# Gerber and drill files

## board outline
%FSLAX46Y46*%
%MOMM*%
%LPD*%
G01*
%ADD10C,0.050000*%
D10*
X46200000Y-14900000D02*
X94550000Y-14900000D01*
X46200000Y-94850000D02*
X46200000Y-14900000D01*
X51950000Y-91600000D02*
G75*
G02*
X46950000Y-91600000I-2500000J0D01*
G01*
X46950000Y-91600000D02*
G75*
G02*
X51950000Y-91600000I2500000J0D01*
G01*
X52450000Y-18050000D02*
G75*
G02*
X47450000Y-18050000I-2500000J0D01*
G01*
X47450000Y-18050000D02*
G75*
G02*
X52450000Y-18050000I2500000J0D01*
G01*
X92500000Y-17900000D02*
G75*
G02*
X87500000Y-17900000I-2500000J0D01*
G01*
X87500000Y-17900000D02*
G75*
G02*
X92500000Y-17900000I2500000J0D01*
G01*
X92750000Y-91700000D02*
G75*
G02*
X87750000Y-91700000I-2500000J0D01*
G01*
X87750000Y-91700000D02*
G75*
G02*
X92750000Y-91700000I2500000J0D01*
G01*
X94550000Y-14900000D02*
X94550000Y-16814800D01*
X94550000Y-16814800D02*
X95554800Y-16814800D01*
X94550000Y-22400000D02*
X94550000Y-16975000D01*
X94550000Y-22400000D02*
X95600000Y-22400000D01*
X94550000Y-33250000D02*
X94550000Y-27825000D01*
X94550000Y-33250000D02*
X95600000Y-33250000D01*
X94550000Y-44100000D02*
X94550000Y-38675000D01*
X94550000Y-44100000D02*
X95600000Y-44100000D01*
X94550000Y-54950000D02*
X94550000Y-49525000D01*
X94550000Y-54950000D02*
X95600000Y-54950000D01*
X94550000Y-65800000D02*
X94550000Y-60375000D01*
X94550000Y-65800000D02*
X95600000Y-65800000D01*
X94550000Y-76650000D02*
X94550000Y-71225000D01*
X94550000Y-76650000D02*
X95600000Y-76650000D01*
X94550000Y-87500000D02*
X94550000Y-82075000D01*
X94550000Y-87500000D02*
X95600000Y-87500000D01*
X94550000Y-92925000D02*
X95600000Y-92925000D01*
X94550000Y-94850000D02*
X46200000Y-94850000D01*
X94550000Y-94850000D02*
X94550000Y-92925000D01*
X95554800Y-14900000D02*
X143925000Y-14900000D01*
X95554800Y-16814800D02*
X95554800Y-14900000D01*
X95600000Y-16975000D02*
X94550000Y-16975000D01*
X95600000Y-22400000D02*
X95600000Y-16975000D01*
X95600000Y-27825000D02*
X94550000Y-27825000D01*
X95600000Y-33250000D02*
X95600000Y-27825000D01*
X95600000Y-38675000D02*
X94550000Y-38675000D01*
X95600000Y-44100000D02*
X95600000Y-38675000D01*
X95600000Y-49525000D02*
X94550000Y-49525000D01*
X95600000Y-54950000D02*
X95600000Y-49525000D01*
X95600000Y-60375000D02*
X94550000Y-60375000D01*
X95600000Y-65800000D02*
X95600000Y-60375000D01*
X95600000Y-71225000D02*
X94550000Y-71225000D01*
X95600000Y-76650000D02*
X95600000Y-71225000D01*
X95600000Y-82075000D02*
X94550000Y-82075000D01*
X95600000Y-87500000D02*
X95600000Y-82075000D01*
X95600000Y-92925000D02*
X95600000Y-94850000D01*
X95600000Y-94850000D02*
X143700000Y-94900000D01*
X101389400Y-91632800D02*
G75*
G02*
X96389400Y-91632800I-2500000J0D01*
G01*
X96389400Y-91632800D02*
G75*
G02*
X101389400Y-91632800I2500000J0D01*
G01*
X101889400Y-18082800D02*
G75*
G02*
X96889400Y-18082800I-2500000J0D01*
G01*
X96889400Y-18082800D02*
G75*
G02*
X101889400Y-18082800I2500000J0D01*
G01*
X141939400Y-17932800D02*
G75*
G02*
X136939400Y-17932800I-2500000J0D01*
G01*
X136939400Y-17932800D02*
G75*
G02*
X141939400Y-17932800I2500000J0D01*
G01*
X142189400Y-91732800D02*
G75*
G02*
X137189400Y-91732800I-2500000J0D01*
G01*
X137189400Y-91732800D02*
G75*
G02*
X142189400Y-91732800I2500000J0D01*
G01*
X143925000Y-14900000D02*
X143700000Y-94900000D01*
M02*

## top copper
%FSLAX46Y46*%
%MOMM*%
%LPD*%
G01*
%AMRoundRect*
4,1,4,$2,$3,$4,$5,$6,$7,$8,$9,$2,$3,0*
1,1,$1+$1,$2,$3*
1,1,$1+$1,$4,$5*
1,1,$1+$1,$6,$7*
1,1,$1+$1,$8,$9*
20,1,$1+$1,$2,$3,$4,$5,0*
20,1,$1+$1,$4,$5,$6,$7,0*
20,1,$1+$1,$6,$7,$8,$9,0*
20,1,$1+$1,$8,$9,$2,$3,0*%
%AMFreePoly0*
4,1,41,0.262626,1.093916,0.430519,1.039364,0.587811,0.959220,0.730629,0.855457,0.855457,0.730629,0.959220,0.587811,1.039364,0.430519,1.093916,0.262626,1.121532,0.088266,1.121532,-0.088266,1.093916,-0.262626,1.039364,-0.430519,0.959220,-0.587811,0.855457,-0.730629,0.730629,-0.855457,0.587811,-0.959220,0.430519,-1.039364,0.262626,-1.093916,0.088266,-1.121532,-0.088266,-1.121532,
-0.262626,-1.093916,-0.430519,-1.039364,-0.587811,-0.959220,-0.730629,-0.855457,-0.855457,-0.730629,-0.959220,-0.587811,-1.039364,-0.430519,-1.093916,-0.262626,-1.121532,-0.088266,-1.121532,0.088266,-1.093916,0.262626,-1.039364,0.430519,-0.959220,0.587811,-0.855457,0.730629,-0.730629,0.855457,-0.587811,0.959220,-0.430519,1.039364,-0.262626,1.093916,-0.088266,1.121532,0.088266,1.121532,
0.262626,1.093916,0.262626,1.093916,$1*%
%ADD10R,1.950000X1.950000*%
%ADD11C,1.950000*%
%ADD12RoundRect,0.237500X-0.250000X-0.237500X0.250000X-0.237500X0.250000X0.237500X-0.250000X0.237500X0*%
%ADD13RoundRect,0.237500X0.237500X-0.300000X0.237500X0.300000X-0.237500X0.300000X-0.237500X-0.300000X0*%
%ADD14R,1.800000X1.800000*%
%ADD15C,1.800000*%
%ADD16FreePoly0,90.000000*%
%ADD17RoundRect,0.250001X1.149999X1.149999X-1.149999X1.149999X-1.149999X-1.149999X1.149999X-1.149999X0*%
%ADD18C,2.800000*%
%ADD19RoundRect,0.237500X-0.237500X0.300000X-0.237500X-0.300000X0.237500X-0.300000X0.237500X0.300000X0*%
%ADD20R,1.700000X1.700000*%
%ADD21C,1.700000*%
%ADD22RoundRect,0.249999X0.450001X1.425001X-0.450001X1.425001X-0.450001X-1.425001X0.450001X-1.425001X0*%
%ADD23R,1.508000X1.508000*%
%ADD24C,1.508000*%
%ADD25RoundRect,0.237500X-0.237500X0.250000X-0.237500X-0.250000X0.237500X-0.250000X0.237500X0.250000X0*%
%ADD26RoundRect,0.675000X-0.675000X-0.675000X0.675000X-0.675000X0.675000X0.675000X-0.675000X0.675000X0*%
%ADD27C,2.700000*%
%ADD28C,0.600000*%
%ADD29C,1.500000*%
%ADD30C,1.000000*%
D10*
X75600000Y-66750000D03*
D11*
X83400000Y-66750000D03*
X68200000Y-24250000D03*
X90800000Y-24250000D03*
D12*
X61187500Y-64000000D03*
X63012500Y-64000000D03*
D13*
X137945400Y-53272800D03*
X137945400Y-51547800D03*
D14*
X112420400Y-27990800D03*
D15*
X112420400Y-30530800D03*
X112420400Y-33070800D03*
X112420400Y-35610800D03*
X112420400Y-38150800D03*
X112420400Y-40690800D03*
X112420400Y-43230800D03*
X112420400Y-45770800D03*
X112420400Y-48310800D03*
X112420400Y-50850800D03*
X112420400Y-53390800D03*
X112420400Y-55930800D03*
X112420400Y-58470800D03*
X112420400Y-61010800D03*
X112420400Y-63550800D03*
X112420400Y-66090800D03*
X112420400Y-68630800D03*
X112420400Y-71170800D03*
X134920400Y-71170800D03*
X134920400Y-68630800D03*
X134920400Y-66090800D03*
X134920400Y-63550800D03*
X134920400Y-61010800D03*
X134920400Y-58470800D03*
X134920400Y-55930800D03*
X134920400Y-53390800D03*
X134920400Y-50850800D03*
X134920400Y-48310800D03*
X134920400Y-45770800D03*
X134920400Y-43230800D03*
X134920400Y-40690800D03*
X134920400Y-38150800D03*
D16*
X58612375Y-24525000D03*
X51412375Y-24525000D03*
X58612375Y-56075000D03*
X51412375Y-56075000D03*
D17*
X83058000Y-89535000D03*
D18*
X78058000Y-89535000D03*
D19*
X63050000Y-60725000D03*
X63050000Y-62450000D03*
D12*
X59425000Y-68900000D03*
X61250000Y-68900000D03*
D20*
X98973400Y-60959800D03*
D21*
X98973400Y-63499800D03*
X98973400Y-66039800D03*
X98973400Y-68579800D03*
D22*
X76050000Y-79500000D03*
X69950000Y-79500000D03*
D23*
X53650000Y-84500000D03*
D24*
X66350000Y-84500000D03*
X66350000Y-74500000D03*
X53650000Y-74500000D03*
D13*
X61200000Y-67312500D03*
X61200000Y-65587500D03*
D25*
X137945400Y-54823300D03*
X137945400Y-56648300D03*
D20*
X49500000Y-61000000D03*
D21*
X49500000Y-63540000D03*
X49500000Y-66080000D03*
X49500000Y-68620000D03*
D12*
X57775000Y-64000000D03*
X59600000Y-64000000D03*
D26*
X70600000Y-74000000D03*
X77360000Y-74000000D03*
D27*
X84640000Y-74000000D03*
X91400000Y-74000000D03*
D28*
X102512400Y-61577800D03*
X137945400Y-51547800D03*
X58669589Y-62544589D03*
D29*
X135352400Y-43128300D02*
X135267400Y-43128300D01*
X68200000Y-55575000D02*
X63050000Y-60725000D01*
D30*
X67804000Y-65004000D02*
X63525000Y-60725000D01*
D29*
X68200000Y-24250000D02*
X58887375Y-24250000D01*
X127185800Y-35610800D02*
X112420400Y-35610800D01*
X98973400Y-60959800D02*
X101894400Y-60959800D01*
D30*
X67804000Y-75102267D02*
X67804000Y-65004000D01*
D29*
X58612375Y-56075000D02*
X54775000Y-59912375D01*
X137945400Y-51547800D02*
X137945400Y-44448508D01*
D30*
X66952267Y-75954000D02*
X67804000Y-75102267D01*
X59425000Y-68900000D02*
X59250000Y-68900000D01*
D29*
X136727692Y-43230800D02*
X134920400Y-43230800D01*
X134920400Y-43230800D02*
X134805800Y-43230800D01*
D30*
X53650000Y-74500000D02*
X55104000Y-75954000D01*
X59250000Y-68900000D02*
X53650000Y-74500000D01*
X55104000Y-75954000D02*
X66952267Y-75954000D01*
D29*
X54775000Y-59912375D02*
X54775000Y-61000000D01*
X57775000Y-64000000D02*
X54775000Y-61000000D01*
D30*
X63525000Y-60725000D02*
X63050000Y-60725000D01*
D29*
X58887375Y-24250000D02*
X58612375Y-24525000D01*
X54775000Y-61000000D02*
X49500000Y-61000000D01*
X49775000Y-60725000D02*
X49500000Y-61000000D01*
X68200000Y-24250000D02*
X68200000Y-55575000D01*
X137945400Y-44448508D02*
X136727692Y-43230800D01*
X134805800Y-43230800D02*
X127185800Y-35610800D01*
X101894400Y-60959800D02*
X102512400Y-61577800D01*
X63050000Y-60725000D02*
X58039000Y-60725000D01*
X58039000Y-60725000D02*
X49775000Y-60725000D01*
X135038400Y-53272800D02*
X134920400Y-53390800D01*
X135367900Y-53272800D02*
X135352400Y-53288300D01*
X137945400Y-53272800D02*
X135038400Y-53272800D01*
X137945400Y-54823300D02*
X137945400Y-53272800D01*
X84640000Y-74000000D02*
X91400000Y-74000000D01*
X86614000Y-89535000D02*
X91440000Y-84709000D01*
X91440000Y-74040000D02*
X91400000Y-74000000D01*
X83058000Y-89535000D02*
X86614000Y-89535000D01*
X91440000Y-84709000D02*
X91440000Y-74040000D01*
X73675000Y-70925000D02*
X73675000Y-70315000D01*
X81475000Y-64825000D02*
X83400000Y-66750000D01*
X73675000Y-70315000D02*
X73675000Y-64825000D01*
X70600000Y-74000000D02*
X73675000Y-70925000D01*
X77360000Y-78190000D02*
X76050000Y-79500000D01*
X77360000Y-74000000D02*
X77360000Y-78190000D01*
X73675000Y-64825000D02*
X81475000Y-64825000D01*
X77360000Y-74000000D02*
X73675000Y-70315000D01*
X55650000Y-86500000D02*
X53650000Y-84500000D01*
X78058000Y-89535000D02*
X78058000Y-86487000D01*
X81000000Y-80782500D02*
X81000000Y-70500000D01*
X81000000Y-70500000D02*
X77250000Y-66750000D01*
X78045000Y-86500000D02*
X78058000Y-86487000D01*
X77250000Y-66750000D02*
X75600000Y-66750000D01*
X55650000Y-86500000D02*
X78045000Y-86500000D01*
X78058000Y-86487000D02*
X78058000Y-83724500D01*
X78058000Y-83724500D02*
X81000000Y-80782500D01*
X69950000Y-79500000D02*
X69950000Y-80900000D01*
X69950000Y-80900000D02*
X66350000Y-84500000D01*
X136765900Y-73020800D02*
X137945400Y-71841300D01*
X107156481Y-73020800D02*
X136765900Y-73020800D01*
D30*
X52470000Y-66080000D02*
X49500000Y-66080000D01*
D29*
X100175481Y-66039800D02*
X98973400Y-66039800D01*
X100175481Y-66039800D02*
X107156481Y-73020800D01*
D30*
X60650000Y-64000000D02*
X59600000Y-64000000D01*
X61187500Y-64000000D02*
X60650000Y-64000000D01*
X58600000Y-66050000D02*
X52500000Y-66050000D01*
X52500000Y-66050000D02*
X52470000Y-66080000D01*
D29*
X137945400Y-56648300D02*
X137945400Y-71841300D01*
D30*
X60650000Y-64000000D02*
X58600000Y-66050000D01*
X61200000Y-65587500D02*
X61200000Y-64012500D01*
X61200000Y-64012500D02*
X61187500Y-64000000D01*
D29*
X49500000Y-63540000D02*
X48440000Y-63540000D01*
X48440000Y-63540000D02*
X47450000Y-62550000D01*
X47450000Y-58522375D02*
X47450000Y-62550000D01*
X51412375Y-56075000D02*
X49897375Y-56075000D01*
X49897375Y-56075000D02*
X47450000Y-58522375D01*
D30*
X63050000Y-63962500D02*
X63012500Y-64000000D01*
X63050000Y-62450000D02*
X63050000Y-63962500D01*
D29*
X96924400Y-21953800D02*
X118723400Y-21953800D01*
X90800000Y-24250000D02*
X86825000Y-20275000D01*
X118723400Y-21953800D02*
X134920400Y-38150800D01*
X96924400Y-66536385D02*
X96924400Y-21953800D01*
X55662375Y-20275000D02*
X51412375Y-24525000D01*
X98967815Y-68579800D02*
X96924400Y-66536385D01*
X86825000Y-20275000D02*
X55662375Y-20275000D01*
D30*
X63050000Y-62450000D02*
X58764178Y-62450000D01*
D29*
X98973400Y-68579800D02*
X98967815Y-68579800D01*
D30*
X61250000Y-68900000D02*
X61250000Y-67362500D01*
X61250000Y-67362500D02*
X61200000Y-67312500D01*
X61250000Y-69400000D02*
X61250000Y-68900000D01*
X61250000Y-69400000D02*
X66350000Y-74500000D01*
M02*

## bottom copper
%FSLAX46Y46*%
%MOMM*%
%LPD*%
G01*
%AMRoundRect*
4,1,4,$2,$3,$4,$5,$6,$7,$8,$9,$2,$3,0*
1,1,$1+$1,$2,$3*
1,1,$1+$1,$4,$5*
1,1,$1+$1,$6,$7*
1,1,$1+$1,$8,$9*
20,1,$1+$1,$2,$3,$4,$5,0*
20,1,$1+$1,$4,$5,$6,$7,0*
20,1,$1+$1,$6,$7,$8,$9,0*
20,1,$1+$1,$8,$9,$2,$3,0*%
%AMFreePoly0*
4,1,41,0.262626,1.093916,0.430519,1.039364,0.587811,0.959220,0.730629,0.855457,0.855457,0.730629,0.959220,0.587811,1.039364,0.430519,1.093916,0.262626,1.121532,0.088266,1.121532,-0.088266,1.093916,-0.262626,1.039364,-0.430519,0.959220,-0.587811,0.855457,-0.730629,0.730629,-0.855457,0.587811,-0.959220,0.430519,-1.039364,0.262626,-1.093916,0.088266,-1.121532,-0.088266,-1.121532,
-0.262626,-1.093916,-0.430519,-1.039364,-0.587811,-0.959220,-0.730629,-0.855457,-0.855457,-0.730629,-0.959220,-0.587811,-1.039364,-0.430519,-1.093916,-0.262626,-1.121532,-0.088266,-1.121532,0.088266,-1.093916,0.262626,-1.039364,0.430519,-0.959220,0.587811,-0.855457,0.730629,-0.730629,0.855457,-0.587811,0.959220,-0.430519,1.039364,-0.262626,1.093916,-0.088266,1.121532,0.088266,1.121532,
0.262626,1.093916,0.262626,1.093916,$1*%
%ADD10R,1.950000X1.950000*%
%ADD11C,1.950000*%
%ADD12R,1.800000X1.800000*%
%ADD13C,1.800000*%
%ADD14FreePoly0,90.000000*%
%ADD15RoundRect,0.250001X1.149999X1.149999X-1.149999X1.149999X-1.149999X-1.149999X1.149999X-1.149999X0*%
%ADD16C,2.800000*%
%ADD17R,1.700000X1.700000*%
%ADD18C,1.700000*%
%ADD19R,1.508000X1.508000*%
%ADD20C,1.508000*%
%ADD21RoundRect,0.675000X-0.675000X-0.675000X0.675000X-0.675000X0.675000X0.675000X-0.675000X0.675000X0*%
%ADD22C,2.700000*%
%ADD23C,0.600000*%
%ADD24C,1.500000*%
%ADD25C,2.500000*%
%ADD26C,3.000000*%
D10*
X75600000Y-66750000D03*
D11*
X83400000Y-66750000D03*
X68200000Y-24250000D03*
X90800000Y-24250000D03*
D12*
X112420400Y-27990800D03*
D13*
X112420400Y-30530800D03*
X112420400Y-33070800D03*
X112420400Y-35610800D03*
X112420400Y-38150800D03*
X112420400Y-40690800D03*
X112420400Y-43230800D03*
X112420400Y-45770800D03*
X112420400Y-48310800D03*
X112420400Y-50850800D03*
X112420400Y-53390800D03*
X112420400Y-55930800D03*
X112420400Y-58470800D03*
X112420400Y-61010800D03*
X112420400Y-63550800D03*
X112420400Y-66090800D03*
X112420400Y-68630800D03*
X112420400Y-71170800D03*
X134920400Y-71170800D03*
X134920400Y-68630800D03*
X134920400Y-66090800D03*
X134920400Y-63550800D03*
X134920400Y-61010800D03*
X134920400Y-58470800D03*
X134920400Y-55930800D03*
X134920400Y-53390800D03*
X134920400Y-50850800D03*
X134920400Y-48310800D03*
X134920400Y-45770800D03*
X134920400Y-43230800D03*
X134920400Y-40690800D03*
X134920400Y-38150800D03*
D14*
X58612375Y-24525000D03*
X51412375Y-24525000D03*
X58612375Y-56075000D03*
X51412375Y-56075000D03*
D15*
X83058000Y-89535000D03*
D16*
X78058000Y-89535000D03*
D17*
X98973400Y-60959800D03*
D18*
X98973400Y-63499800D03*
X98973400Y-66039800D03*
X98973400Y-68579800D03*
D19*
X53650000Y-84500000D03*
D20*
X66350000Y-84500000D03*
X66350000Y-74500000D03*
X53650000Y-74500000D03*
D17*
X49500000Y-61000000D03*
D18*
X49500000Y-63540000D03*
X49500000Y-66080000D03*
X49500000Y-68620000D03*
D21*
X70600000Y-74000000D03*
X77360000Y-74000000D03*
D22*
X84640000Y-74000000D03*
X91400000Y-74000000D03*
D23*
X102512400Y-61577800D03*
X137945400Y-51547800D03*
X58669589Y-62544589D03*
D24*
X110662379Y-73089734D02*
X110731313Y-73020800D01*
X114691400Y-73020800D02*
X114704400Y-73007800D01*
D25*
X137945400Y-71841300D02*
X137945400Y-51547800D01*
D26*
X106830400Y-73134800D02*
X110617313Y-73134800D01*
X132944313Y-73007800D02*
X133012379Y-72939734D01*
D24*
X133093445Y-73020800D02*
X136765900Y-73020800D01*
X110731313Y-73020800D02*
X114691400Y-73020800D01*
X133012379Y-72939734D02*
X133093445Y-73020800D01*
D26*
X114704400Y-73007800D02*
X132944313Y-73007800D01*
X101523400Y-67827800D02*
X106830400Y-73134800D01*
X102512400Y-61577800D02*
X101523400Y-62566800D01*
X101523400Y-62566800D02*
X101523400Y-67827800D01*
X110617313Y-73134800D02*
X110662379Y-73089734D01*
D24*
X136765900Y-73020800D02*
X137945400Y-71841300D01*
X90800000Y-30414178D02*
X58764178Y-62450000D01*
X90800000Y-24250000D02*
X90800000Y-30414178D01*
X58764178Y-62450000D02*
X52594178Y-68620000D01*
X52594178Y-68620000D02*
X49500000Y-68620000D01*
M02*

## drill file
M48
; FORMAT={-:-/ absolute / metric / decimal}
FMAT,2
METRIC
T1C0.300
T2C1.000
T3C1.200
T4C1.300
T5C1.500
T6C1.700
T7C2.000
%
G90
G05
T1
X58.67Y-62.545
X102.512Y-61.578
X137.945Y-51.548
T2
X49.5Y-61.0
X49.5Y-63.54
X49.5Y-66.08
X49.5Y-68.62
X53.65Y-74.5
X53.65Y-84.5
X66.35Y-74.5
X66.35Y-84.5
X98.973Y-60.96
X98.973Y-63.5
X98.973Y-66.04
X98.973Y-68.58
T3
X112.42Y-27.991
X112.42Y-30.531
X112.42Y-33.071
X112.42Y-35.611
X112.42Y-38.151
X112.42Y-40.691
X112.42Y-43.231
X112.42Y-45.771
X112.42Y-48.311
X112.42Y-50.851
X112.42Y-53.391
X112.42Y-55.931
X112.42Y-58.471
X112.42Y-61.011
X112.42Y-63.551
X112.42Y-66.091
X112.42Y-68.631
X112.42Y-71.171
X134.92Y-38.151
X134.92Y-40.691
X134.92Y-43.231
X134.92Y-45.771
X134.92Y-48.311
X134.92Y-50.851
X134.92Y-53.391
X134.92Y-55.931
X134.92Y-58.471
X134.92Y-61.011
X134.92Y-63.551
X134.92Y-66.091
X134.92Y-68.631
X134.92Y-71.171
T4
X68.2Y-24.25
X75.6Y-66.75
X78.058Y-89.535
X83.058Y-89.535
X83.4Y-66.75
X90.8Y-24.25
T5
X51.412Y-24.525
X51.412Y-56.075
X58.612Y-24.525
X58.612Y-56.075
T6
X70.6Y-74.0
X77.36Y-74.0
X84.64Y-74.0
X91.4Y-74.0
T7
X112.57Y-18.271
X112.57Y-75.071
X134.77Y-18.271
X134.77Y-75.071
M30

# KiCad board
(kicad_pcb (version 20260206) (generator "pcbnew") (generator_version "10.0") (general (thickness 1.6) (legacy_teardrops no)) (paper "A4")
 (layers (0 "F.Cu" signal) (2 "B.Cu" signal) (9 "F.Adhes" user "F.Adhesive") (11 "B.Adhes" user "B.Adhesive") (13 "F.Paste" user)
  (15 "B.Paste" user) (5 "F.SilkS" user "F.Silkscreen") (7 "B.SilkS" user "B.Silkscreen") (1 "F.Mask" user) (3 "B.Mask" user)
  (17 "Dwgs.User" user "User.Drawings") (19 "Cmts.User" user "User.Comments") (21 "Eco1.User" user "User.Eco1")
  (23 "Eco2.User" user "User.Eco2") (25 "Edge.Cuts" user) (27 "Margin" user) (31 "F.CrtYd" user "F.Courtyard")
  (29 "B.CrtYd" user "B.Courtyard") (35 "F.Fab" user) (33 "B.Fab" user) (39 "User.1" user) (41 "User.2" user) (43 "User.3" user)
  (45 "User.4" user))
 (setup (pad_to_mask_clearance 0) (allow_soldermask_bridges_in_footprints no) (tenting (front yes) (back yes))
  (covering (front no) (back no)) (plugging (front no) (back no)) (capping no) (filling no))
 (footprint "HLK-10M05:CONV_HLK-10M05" (layer "F.Cu") (at 79.5 45.5 90)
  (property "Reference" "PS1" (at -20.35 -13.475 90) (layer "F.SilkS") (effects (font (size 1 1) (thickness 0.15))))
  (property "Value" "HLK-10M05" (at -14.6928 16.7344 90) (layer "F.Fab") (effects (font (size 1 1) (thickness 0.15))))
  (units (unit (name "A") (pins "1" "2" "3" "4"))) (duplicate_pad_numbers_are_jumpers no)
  (pad "1" thru_hole rect (at -21.25 -3.9 90) (size 1.95 1.95) (drill 1.3) (layers "*.Cu" "*.Mask") (remove_unused_layers no) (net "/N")
   (solder_mask_margin 0.102))
  (pad "2" thru_hole circle (at -21.25 3.9 90) (size 1.95 1.95) (drill 1.3) (layers "*.Cu" "*.Mask") (remove_unused_layers no)
   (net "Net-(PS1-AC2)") (solder_mask_margin 0.102))
  (pad "3" thru_hole circle (at 21.25 -11.3 90) (size 1.95 1.95) (drill 1.3) (layers "*.Cu" "*.Mask") (remove_unused_layers no) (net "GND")
   (solder_mask_margin 0.102))
  (pad "4" thru_hole circle (at 21.25 11.3 90) (size 1.95 1.95) (drill 1.3) (layers "*.Cu" "*.Mask") (remove_unused_layers no) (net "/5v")
   (solder_mask_margin 0.102)))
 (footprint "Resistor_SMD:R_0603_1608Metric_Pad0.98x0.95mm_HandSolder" (layer "F.Cu") (at 62.1 64)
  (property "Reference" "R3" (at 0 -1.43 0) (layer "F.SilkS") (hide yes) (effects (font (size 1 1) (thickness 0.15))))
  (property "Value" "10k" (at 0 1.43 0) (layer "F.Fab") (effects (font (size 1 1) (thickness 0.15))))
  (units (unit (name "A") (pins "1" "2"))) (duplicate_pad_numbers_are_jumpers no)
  (pad "1" smd roundrect (at -0.9125 0) (size 0.975 0.95) (layers "F.Cu" "F.Mask" "F.Paste") (roundrect_rratio 0.25) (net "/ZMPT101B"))
  (pad "2" smd roundrect (at 0.9125 0) (size 0.975 0.95) (layers "F.Cu" "F.Mask" "F.Paste") (roundrect_rratio 0.25) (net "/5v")))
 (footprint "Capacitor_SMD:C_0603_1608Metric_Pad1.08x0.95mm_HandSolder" (layer "F.Cu") (at 137.9454 52.4103 90)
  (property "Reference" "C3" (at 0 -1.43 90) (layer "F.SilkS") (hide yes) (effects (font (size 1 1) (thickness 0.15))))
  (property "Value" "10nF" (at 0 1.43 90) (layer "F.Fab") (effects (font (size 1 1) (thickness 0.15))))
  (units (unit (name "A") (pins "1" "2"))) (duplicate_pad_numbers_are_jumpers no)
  (pad "1" smd roundrect (at -0.8625 0 90) (size 1.075 0.95) (layers "F.Cu" "F.Mask" "F.Paste") (roundrect_rratio 0.25) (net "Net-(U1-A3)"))
  (pad "2" smd roundrect (at 0.8625 0 90) (size 1.075 0.95) (layers "F.Cu" "F.Mask" "F.Paste") (roundrect_rratio 0.25) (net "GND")))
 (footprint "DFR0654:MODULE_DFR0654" (layer "F.Cu") (at 123.6704 46.6708)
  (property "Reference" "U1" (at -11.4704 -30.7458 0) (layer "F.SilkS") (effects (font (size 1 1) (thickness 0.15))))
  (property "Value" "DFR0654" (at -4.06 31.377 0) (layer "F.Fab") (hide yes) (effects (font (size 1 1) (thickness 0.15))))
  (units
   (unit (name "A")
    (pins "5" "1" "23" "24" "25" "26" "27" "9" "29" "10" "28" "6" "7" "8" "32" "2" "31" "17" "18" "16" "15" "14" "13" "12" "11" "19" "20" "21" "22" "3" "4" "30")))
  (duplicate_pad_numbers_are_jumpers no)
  (pad "" np_thru_hole circle (at -11.1 -28.4) (size 2 2) (drill 2) (layers "*.Cu" "*.Mask"))
  (pad "" np_thru_hole circle (at -11.1 28.4) (size 2 2) (drill 2) (layers "*.Cu" "*.Mask"))
  (pad "" np_thru_hole circle (at 11.1 -28.4) (size 2 2) (drill 2) (layers "*.Cu" "*.Mask"))
  (pad "" np_thru_hole circle (at 11.1 28.4) (size 2 2) (drill 2) (layers "*.Cu" "*.Mask"))
  (pad "1" thru_hole rect (at -11.25 -18.68) (size 1.8 1.8) (drill 1.2) (layers "*.Cu" "*.Mask") (remove_unused_layers no)
   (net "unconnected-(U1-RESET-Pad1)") (solder_mask_margin 0.102))
  (pad "2" thru_hole circle (at -11.25 -16.14) (size 1.8 1.8) (drill 1.2) (layers "*.Cu" "*.Mask") (remove_unused_layers no) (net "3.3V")
   (solder_mask_margin 0.102))
  (pad "3" thru_hole circle (at -11.25 -13.6) (size 1.8 1.8) (drill 1.2) (layers "*.Cu" "*.Mask") (remove_unused_layers no)
   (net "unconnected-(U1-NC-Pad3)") (solder_mask_margin 0.102))
  (pad "4" thru_hole circle (at -11.25 -11.06) (size 1.8 1.8) (drill 1.2) (layers "*.Cu" "*.Mask") (remove_unused_layers no) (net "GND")
   (solder_mask_margin 0.102))
  (pad "5" thru_hole circle (at -11.25 -8.52) (size 1.8 1.8) (drill 1.2) (layers "*.Cu" "*.Mask") (remove_unused_layers no)
   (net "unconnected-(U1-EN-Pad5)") (solder_mask_margin 0.102))
  (pad "6" thru_hole circle (at -11.25 -5.98) (size 1.8 1.8) (drill 1.2) (layers "*.Cu" "*.Mask") (remove_unused_layers no)
   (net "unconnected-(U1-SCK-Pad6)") (solder_mask_margin 0.102))
  (pad "7" thru_hole circle (at -11.25 -3.44) (size 1.8 1.8) (drill 1.2) (layers "*.Cu" "*.Mask") (remove_unused_layers no)
   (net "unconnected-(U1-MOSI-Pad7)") (solder_mask_margin 0.102))
  (pad "8" thru_hole circle (at -11.25 -0.9) (size 1.8 1.8) (drill 1.2) (layers "*.Cu" "*.Mask") (remove_unused_layers no)
   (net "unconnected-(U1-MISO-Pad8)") (solder_mask_margin 0.102))
  (pad "9" thru_hole circle (at -11.25 1.64) (size 1.8 1.8) (drill 1.2) (layers "*.Cu" "*.Mask") (remove_unused_layers no)
   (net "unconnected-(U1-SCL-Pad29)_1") (solder_mask_margin 0.102))
  (pad "10" thru_hole circle (at -11.25 4.18) (size 1.8 1.8) (drill 1.2) (layers "*.Cu" "*.Mask") (remove_unused_layers no)
   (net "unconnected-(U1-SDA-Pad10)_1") (solder_mask_margin 0.102))
  (pad "11" thru_hole circle (at -11.25 6.72) (size 1.8 1.8) (drill 1.2) (layers "*.Cu" "*.Mask") (remove_unused_layers no)
   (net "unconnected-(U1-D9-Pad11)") (solder_mask_margin 0.102))
  (pad "12" thru_hole circle (at -11.25 9.26) (size 1.8 1.8) (drill 1.2) (layers "*.Cu" "*.Mask") (remove_unused_layers no)
   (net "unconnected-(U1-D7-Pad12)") (solder_mask_margin 0.102))
  (pad "13" thru_hole circle (at -11.25 11.8) (size 1.8 1.8) (drill 1.2) (layers "*.Cu" "*.Mask") (remove_unused_layers no)
   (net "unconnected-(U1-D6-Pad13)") (solder_mask_margin 0.102))
  (pad "14" thru_hole circle (at -11.25 14.34) (size 1.8 1.8) (drill 1.2) (layers "*.Cu" "*.Mask") (remove_unused_layers no)
   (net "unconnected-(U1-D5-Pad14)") (solder_mask_margin 0.102))
  (pad "15" thru_hole circle (at -11.25 16.88) (size 1.8 1.8) (drill 1.2) (layers "*.Cu" "*.Mask") (remove_unused_layers no)
   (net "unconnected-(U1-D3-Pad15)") (solder_mask_margin 0.102))
  (pad "16" thru_hole circle (at -11.25 19.42) (size 1.8 1.8) (drill 1.2) (layers "*.Cu" "*.Mask") (remove_unused_layers no)
   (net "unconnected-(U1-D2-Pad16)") (solder_mask_margin 0.102))
  (pad "17" thru_hole circle (at -11.25 21.96) (size 1.8 1.8) (drill 1.2) (layers "*.Cu" "*.Mask") (remove_unused_layers no)
   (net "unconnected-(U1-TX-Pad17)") (solder_mask_margin 0.102))
  (pad "18" thru_hole circle (at -11.25 24.5) (size 1.8 1.8) (drill 1.2) (layers "*.Cu" "*.Mask") (remove_unused_layers no)
   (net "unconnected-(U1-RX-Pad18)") (solder_mask_margin 0.102))
  (pad "19" thru_hole circle (at 11.25 24.5) (size 1.8 1.8) (drill 1.2) (layers "*.Cu" "*.Mask") (remove_unused_layers no)
   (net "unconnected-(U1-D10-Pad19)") (solder_mask_margin 0.102))
  (pad "20" thru_hole circle (at 11.25 21.96) (size 1.8 1.8) (drill 1.2) (layers "*.Cu" "*.Mask") (remove_unused_layers no)
   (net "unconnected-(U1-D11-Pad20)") (solder_mask_margin 0.102))
  (pad "21" thru_hole circle (at 11.25 19.42) (size 1.8 1.8) (drill 1.2) (layers "*.Cu" "*.Mask") (remove_unused_layers no)
   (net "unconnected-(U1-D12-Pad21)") (solder_mask_margin 0.102))
  (pad "22" thru_hole circle (at 11.25 16.88) (size 1.8 1.8) (drill 1.2) (layers "*.Cu" "*.Mask") (remove_unused_layers no)
   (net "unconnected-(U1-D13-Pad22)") (solder_mask_margin 0.102))
  (pad "23" thru_hole circle (at 11.25 14.34) (size 1.8 1.8) (drill 1.2) (layers "*.Cu" "*.Mask") (remove_unused_layers no)
   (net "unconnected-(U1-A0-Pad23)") (solder_mask_margin 0.102))
  (pad "24" thru_hole circle (at 11.25 11.8) (size 1.8 1.8) (drill 1.2) (layers "*.Cu" "*.Mask") (remove_unused_layers no)
   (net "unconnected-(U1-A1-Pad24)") (solder_mask_margin 0.102))
  (pad "25" thru_hole circle (at 11.25 9.26) (size 1.8 1.8) (drill 1.2) (layers "*.Cu" "*.Mask") (remove_unused_layers no)
   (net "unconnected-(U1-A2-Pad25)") (solder_mask_margin 0.102))
  (pad "26" thru_hole circle (at 11.25 6.72) (size 1.8 1.8) (drill 1.2) (layers "*.Cu" "*.Mask") (remove_unused_layers no)
   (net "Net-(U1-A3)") (solder_mask_margin 0.102))
  (pad "27" thru_hole circle (at 11.25 4.18) (size 1.8 1.8) (drill 1.2) (layers "*.Cu" "*.Mask") (remove_unused_layers no)
   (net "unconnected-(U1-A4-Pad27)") (solder_mask_margin 0.102))
  (pad "28" thru_hole circle (at 11.25 1.64) (size 1.8 1.8) (drill 1.2) (layers "*.Cu" "*.Mask") (remove_unused_layers no)
   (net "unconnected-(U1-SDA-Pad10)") (solder_mask_margin 0.102))
  (pad "29" thru_hole circle (at 11.25 -0.9) (size 1.8 1.8) (drill 1.2) (layers "*.Cu" "*.Mask") (remove_unused_layers no)
   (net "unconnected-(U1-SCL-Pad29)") (solder_mask_margin 0.102))
  (pad "30" thru_hole circle (at 11.25 -3.44) (size 1.8 1.8) (drill 1.2) (layers "*.Cu" "*.Mask") (remove_unused_layers no) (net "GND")
   (solder_mask_margin 0.102))
  (pad "31" thru_hole circle (at 11.25 -5.98) (size 1.8 1.8) (drill 1.2) (layers "*.Cu" "*.Mask") (remove_unused_layers no) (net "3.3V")
   (solder_mask_margin 0.102))
  (pad "32" thru_hole circle (at 11.25 -8.52) (size 1.8 1.8) (drill 1.2) (layers "*.Cu" "*.Mask") (remove_unused_layers no) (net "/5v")
   (solder_mask_margin 0.102)))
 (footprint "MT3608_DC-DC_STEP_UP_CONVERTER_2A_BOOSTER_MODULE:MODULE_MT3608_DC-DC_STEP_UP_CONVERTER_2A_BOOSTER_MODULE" (layer "F.Cu")
  (at 55.012375 40.3 90)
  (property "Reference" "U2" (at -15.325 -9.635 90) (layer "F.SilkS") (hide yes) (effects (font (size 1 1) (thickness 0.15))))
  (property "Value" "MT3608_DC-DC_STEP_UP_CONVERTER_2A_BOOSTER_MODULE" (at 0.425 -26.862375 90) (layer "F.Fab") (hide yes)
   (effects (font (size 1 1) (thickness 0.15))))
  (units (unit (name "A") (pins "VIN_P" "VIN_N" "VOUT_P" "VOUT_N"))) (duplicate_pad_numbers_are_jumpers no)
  (pad "VIN_N" thru_hole custom (at 15.775 3.6 90) (size 2.25 2.25) (drill 1.5) (layers "*.Cu") (remove_unused_layers no) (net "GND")
   (thermal_bridge_angle 90) (options (clearance outline) (anchor circle)) (primitives))
  (pad "VIN_P" thru_hole custom (at 15.775 -3.6 90) (size 2.25 2.25) (drill 1.5) (layers "*.Cu") (remove_unused_layers no) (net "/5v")
   (thermal_bridge_angle 90) (options (clearance outline) (anchor circle)) (primitives))
  (pad "VOUT_N" thru_hole custom (at -15.775 3.6 90) (size 2.25 2.25) (drill 1.5) (layers "*.Cu") (remove_unused_layers no) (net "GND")
   (thermal_bridge_angle 90) (options (clearance outline) (anchor circle)) (primitives))
  (pad "VOUT_P" thru_hole custom (at -15.775 -3.6 90) (size 2.25 2.25) (drill 1.5) (layers "*.Cu") (remove_unused_layers no) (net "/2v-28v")
   (thermal_bridge_angle 90) (options (clearance outline) (anchor circle)) (primitives)))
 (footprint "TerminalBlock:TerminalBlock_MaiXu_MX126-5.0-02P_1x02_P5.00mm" (layer "F.Cu") (at 83.058 89.535 180)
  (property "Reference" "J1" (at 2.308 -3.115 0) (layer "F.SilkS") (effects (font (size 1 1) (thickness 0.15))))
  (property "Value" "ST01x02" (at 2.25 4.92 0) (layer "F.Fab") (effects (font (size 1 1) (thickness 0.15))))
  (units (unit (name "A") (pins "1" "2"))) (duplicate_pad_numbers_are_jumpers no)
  (pad "1" thru_hole roundrect (at 0 0 180) (size 2.8 2.8) (drill 1.3) (layers "*.Cu" "*.Mask") (remove_unused_layers no)
   (roundrect_rratio 0.089286) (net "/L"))
  (pad "2" thru_hole circle (at 5 0 180) (size 2.8 2.8) (drill 1.3) (layers "*.Cu" "*.Mask") (remove_unused_layers no) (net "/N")))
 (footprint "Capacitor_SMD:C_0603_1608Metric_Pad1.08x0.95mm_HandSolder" (layer "F.Cu") (at 63.05 61.5875 -90)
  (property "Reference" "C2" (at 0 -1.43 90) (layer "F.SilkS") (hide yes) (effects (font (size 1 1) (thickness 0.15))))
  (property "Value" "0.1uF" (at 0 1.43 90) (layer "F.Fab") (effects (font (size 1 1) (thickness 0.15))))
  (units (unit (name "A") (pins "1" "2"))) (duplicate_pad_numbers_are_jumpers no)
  (pad "1" smd roundrect (at -0.8625 0 270) (size 1.075 0.95) (layers "F.Cu" "F.Mask" "F.Paste") (roundrect_rratio 0.25) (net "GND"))
  (pad "2" smd roundrect (at 0.8625 0 270) (size 1.075 0.95) (layers "F.Cu" "F.Mask" "F.Paste") (roundrect_rratio 0.25) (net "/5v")))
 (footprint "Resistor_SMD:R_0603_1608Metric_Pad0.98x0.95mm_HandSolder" (layer "F.Cu") (at 60.3375 68.9)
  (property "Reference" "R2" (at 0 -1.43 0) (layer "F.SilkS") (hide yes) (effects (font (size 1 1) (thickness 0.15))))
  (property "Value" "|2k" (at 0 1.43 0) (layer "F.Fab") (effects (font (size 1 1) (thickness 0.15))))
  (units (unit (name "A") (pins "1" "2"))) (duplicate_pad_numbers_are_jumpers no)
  (pad "1" smd roundrect (at -0.9125 0) (size 0.975 0.95) (layers "F.Cu" "F.Mask" "F.Paste") (roundrect_rratio 0.25) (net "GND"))
  (pad "2" smd roundrect (at 0.9125 0) (size 0.975 0.95) (layers "F.Cu" "F.Mask" "F.Paste") (roundrect_rratio 0.25) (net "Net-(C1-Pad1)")))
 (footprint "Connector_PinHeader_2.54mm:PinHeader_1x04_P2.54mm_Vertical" (layer "F.Cu") (at 98.9734 60.9598)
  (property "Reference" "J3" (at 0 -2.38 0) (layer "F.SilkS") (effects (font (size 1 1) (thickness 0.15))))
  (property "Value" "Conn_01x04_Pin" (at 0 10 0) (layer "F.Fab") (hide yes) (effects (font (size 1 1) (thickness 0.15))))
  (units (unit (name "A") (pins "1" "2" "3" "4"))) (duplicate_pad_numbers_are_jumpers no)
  (pad "1" thru_hole rect (at 0 0) (size 1.7 1.7) (drill 1) (layers "*.Cu" "*.Mask") (remove_unused_layers no) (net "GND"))
  (pad "2" thru_hole circle (at 0 2.54) (size 1.7 1.7) (drill 1) (layers "*.Cu" "*.Mask") (remove_unused_layers no)
   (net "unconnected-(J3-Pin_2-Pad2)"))
  (pad "3" thru_hole circle (at 0 5.08) (size 1.7 1.7) (drill 1) (layers "*.Cu" "*.Mask") (remove_unused_layers no) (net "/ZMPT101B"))
  (pad "4" thru_hole circle (at 0 7.62) (size 1.7 1.7) (drill 1) (layers "*.Cu" "*.Mask") (remove_unused_layers no) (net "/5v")))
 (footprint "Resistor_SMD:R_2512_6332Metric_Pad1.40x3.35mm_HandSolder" (layer "F.Cu") (at 73 79.5 180)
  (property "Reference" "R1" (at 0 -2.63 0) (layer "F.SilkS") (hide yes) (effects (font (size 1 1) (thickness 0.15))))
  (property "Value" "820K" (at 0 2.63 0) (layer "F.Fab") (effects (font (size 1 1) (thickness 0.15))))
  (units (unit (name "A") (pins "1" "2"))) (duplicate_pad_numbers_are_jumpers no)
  (pad "1" smd roundrect (at -3.05 0 180) (size 1.4 3.35) (layers "F.Cu" "F.Mask" "F.Paste") (roundrect_rratio 0.178571)
   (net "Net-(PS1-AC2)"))
  (pad "2" smd roundrect (at 3.05 0 180) (size 1.4 3.35) (layers "F.Cu" "F.Mask" "F.Paste") (roundrect_rratio 0.178571)
   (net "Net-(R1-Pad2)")))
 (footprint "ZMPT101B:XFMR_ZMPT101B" (layer "F.Cu") (at 60 79.5 90)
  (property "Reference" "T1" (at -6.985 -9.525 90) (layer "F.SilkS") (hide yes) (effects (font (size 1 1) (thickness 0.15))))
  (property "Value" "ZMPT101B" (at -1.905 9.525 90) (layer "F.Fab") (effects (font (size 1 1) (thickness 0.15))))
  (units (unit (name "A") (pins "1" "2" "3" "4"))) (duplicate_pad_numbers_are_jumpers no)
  (pad "1" thru_hole rect (at -5 -6.35 90) (size 1.508 1.508) (drill 1) (layers "*.Cu" "*.Mask") (remove_unused_layers no) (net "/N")
   (solder_mask_margin 0.102))
  (pad "2" thru_hole circle (at -5 6.35 90) (size 1.508 1.508) (drill 1) (layers "*.Cu" "*.Mask") (remove_unused_layers no)
   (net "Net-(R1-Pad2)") (solder_mask_margin 0.102))
  (pad "3" thru_hole circle (at 5 6.35 90) (size 1.508 1.508) (drill 1) (layers "*.Cu" "*.Mask") (remove_unused_layers no)
   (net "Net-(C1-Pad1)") (solder_mask_margin 0.102))
  (pad "4" thru_hole circle (at 5 -6.35 90) (size 1.508 1.508) (drill 1) (layers "*.Cu" "*.Mask") (remove_unused_layers no) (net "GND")
   (solder_mask_margin 0.102)))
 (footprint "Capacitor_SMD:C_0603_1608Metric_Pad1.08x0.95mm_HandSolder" (layer "F.Cu") (at 61.2 66.45 90)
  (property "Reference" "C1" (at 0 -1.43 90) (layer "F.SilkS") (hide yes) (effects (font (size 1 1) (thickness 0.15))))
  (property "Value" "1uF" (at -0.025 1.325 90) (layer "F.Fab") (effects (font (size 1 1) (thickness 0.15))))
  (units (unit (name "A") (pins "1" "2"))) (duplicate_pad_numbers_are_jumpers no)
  (pad "1" smd roundrect (at -0.8625 0 90) (size 1.075 0.95) (layers "F.Cu" "F.Mask" "F.Paste") (roundrect_rratio 0.25)
   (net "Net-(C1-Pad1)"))
  (pad "2" smd roundrect (at 0.8625 0 90) (size 1.075 0.95) (layers "F.Cu" "F.Mask" "F.Paste") (roundrect_rratio 0.25) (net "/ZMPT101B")))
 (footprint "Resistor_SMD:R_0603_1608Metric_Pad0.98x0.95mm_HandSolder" (layer "F.Cu") (at 137.9454 55.7358 -90)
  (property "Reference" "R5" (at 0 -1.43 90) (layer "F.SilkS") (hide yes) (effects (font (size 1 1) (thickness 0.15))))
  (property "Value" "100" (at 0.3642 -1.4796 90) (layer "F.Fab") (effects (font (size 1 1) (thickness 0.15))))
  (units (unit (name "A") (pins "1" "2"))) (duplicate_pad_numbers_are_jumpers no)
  (pad "1" smd roundrect (at -0.9125 0 270) (size 0.975 0.95) (layers "F.Cu" "F.Mask" "F.Paste") (roundrect_rratio 0.25) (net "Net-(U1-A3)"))
  (pad "2" smd roundrect (at 0.9125 0 270) (size 0.975 0.95) (layers "F.Cu" "F.Mask" "F.Paste") (roundrect_rratio 0.25) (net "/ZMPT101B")))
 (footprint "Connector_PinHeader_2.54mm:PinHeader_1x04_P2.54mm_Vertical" (layer "F.Cu") (at 49.5 61)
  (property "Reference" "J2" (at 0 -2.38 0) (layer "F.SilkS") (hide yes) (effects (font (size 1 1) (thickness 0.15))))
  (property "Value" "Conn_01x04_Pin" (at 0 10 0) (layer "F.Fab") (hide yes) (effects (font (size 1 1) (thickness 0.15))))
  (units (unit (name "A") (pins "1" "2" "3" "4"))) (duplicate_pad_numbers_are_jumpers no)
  (pad "1" thru_hole rect (at 0 0) (size 1.7 1.7) (drill 1) (layers "*.Cu" "*.Mask") (remove_unused_layers no) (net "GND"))
  (pad "2" thru_hole circle (at 0 2.54) (size 1.7 1.7) (drill 1) (layers "*.Cu" "*.Mask") (remove_unused_layers no) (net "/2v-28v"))
  (pad "3" thru_hole circle (at 0 5.08) (size 1.7 1.7) (drill 1) (layers "*.Cu" "*.Mask") (remove_unused_layers no) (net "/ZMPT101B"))
  (pad "4" thru_hole circle (at 0 7.62) (size 1.7 1.7) (drill 1) (layers "*.Cu" "*.Mask") (remove_unused_layers no) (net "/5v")))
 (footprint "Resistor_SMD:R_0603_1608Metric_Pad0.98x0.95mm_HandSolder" (layer "F.Cu") (at 58.6875 64)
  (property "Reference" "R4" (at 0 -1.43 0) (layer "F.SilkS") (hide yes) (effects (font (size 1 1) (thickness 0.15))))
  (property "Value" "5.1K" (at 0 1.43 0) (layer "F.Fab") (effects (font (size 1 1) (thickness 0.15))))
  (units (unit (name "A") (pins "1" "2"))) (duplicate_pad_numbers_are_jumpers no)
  (pad "1" smd roundrect (at -0.9125 0) (size 0.975 0.95) (layers "F.Cu" "F.Mask" "F.Paste") (roundrect_rratio 0.25) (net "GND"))
  (pad "2" smd roundrect (at 0.9125 0) (size 0.975 0.95) (layers "F.Cu" "F.Mask" "F.Paste") (roundrect_rratio 0.25) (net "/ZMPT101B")))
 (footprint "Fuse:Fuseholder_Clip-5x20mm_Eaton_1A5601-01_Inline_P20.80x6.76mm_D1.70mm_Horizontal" (layer "F.Cu") (at 70.6 74)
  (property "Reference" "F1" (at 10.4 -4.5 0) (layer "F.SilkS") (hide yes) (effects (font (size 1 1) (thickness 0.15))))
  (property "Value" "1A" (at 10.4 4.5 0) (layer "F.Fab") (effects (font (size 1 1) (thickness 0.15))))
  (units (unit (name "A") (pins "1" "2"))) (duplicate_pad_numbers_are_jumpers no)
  (pad "1" thru_hole roundrect (at 0 0) (size 2.7 2.7) (drill 1.7) (layers "*.Cu" "*.Mask") (remove_unused_layers no)
   (roundrect_rratio 0.25) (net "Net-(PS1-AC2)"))
  (pad "1" thru_hole roundrect (at 6.76 0) (size 2.7 2.7) (drill 1.7) (layers "*.Cu" "*.Mask") (remove_unused_layers no)
   (roundrect_rratio 0.25) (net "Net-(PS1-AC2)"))
  (pad "2" thru_hole circle (at 14.04 0) (size 2.7 2.7) (drill 1.7) (layers "*.Cu" "*.Mask") (remove_unused_layers no) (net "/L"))
  (pad "2" thru_hole circle (at 20.8 0) (size 2.7 2.7) (drill 1.7) (layers "*.Cu" "*.Mask") (remove_unused_layers no) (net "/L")))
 (gr_line (start 46.2 14.9) (end 94.55 14.9) (stroke (width 0.05) (type default)) (layer "Edge.Cuts"))
 (gr_line (start 46.2 94.85) (end 46.2 14.9) (stroke (width 0.05) (type default)) (layer "Edge.Cuts"))
 (gr_circle (center 49.45 91.6) (end 51.95 91.6) (stroke (width 0.05) (type default)) (fill no) (layer "Edge.Cuts"))
 (gr_circle (center 49.95 18.05) (end 52.45 18.05) (stroke (width 0.05) (type default)) (fill no) (layer "Edge.Cuts"))
 (gr_circle (center 90 17.9) (end 92.5 17.9) (stroke (width 0.05) (type default)) (fill no) (layer "Edge.Cuts"))
 (gr_circle (center 90.25 91.7) (end 92.75 91.7) (stroke (width 0.05) (type default)) (fill no) (layer "Edge.Cuts"))
 (gr_line (start 94.55 14.9) (end 94.55 16.8148) (stroke (width 0.05) (type default)) (layer "Edge.Cuts"))
 (gr_line (start 94.55 16.8148) (end 95.5548 16.8148) (stroke (width 0.05) (type default)) (layer "Edge.Cuts"))
 (gr_line (start 94.55 22.4) (end 94.55 16.975) (stroke (width 0.05) (type default)) (layer "Edge.Cuts"))
 (gr_line (start 94.55 22.4) (end 95.6 22.4) (stroke (width 0.05) (type default)) (layer "Edge.Cuts"))
 (gr_line (start 94.55 33.25) (end 94.55 27.825) (stroke (width 0.05) (type default)) (layer "Edge.Cuts"))
 (gr_line (start 94.55 33.25) (end 95.6 33.25) (stroke (width 0.05) (type default)) (layer "Edge.Cuts"))
 (gr_line (start 94.55 44.1) (end 94.55 38.675) (stroke (width 0.05) (type default)) (layer "Edge.Cuts"))
 (gr_line (start 94.55 44.1) (end 95.6 44.1) (stroke (width 0.05) (type default)) (layer "Edge.Cuts"))
 (gr_line (start 94.55 54.95) (end 94.55 49.525) (stroke (width 0.05) (type default)) (layer "Edge.Cuts"))
 (gr_line (start 94.55 54.95) (end 95.6 54.95) (stroke (width 0.05) (type default)) (layer "Edge.Cuts"))
 (gr_line (start 94.55 65.8) (end 94.55 60.375) (stroke (width 0.05) (type default)) (layer "Edge.Cuts"))
 (gr_line (start 94.55 65.8) (end 95.6 65.8) (stroke (width 0.05) (type default)) (layer "Edge.Cuts"))
 (gr_line (start 94.55 76.65) (end 94.55 71.225) (stroke (width 0.05) (type default)) (layer "Edge.Cuts"))
 (gr_line (start 94.55 76.65) (end 95.6 76.65) (stroke (width 0.05) (type default)) (layer "Edge.Cuts"))
 (gr_line (start 94.55 87.5) (end 94.55 82.075) (stroke (width 0.05) (type default)) (layer "Edge.Cuts"))
 (gr_line (start 94.55 87.5) (end 95.6 87.5) (stroke (width 0.05) (type default)) (layer "Edge.Cuts"))
 (gr_line (start 94.55 92.925) (end 95.6 92.925) (stroke (width 0.05) (type default)) (layer "Edge.Cuts"))
 (gr_line (start 94.55 94.85) (end 46.2 94.85) (stroke (width 0.05) (type default)) (layer "Edge.Cuts"))
 (gr_line (start 94.55 94.85) (end 94.55 92.925) (stroke (width 0.05) (type default)) (layer "Edge.Cuts"))
 (gr_line (start 95.5548 14.9) (end 143.925 14.9) (stroke (width 0.05) (type default)) (layer "Edge.Cuts"))
 (gr_line (start 95.5548 16.8148) (end 95.5548 14.9) (stroke (width 0.05) (type default)) (layer "Edge.Cuts"))
 (gr_line (start 95.6 16.975) (end 94.55 16.975) (stroke (width 0.05) (type default)) (layer "Edge.Cuts"))
 (gr_line (start 95.6 22.4) (end 95.6 16.975) (stroke (width 0.05) (type default)) (layer "Edge.Cuts"))
 (gr_line (start 95.6 27.825) (end 94.55 27.825) (stroke (width 0.05) (type default)) (layer "Edge.Cuts"))
 (gr_line (start 95.6 33.25) (end 95.6 27.825) (stroke (width 0.05) (type default)) (layer "Edge.Cuts"))
 (gr_line (start 95.6 38.675) (end 94.55 38.675) (stroke (width 0.05) (type default)) (layer "Edge.Cuts"))
 (gr_line (start 95.6 44.1) (end 95.6 38.675) (stroke (width 0.05) (type default)) (layer "Edge.Cuts"))
 (gr_line (start 95.6 49.525) (end 94.55 49.525) (stroke (width 0.05) (type default)) (layer "Edge.Cuts"))
 (gr_line (start 95.6 54.95) (end 95.6 49.525) (stroke (width 0.05) (type default)) (layer "Edge.Cuts"))
 (gr_line (start 95.6 60.375) (end 94.55 60.375) (stroke (width 0.05) (type default)) (layer "Edge.Cuts"))
 (gr_line (start 95.6 65.8) (end 95.6 60.375) (stroke (width 0.05) (type default)) (layer "Edge.Cuts"))
 (gr_line (start 95.6 71.225) (end 94.55 71.225) (stroke (width 0.05) (type default)) (layer "Edge.Cuts"))
 (gr_line (start 95.6 76.65) (end 95.6 71.225) (stroke (width 0.05) (type default)) (layer "Edge.Cuts"))
 (gr_line (start 95.6 82.075) (end 94.55 82.075) (stroke (width 0.05) (type default)) (layer "Edge.Cuts"))
 (gr_line (start 95.6 87.5) (end 95.6 82.075) (stroke (width 0.05) (type default)) (layer "Edge.Cuts"))
 (gr_line (start 95.6 92.925) (end 95.6 94.85) (stroke (width 0.05) (type default)) (layer "Edge.Cuts"))
 (gr_line (start 95.6 94.85) (end 143.7 94.9) (stroke (width 0.05) (type default)) (layer "Edge.Cuts"))
 (gr_circle (center 98.8894 91.6328) (end 101.3894 91.6328) (stroke (width 0.05) (type default)) (fill no) (layer "Edge.Cuts"))
 (gr_circle (center 99.3894 18.0828) (end 101.8894 18.0828) (stroke (width 0.05) (type default)) (fill no) (layer "Edge.Cuts"))
 (gr_circle (center 139.4394 17.9328) (end 141.9394 17.9328) (stroke (width 0.05) (type default)) (fill no) (layer "Edge.Cuts"))
 (gr_circle (center 139.6894 91.7328) (end 142.1894 91.7328) (stroke (width 0.05) (type default)) (fill no) (layer "Edge.Cuts"))
 (gr_line (start 143.925 14.9) (end 143.7 94.9) (stroke (width 0.05) (type default)) (layer "Edge.Cuts"))
 (segment (start 135.3524 43.1283) (end 135.2674 43.1283) (width 1.5) (layer "F.Cu") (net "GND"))
 (segment (start 68.2 55.575) (end 63.05 60.725) (width 1.5) (layer "F.Cu") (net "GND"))
 (segment (start 67.804 65.004) (end 63.525 60.725) (width 1) (layer "F.Cu") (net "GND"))
 (segment (start 68.2 24.25) (end 58.887375 24.25) (width 1.5) (layer "F.Cu") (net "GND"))
 (segment (start 127.1858 35.6108) (end 112.4204 35.6108) (width 1.5) (layer "F.Cu") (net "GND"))
 (segment (start 98.9734 60.9598) (end 101.8944 60.9598) (width 1.5) (layer "F.Cu") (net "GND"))
 (segment (start 67.804 75.102267) (end 67.804 65.004) (width 1) (layer "F.Cu") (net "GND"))
 (segment (start 58.612375 56.075) (end 54.775 59.912375) (width 1.5) (layer "F.Cu") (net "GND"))
 (segment (start 137.9454 51.5478) (end 137.9454 44.448508) (width 1.5) (layer "F.Cu") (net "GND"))
 (segment (start 66.952267 75.954) (end 67.804 75.102267) (width 1) (layer "F.Cu") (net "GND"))
 (segment (start 59.425 68.9) (end 59.25 68.9) (width 1) (layer "F.Cu") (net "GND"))
 (segment (start 136.727692 43.2308) (end 134.9204 43.2308) (width 1.5) (layer "F.Cu") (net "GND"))
 (segment (start 134.9204 43.2308) (end 134.8058 43.2308) (width 1.5) (layer "F.Cu") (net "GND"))
 (segment (start 53.65 74.5) (end 55.104 75.954) (width 1) (layer "F.Cu") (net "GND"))
 (segment (start 59.25 68.9) (end 53.65 74.5) (width 1) (layer "F.Cu") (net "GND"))
 (segment (start 55.104 75.954) (end 66.952267 75.954) (width 1) (layer "F.Cu") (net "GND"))
 (segment (start 54.775 59.912375) (end 54.775 61) (width 1.5) (layer "F.Cu") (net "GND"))
 (segment (start 57.775 64) (end 54.775 61) (width 1.5) (layer "F.Cu") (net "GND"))
 (segment (start 63.525 60.725) (end 63.05 60.725) (width 1) (layer "F.Cu") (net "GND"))
 (segment (start 58.887375 24.25) (end 58.612375 24.525) (width 1.5) (layer "F.Cu") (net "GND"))
 (segment (start 54.775 61) (end 49.5 61) (width 1.5) (layer "F.Cu") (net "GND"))
 (segment (start 49.775 60.725) (end 49.5 61) (width 1.5) (layer "F.Cu") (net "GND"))
 (segment (start 68.2 24.25) (end 68.2 55.575) (width 1.5) (layer "F.Cu") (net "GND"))
 (segment (start 137.9454 44.448508) (end 136.727692 43.2308) (width 1.5) (layer "F.Cu") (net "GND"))
 (segment (start 134.8058 43.2308) (end 127.1858 35.6108) (width 1.5) (layer "F.Cu") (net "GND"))
 (segment (start 101.8944 60.9598) (end 102.5124 61.5778) (width 1.5) (layer "F.Cu") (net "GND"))
 (segment (start 63.05 60.725) (end 58.039 60.725) (width 1.5) (layer "F.Cu") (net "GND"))
 (segment (start 58.039 60.725) (end 49.775 60.725) (width 1.5) (layer "F.Cu") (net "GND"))
 (via (at 102.5124 61.5778) (size 0.6) (drill 0.3) (layers "F.Cu" "B.Cu") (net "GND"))
 (via (at 137.9454 51.5478) (size 0.6) (drill 0.3) (layers "F.Cu" "B.Cu") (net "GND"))
 (segment (start 110.662379 73.089734) (end 110.731313 73.0208) (width 1.5) (layer "B.Cu") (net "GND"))
 (segment (start 114.6914 73.0208) (end 114.7044 73.0078) (width 1.5) (layer "B.Cu") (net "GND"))
 (segment (start 137.9454 71.8413) (end 137.9454 51.5478) (width 2.5) (layer "B.Cu") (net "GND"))
 (segment (start 106.8304 73.1348) (end 110.617313 73.1348) (width 3) (layer "B.Cu") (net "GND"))
 (segment (start 132.944313 73.0078) (end 133.012379 72.939734) (width 3) (layer "B.Cu") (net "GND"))
 (segment (start 133.093445 73.0208) (end 136.7659 73.0208) (width 1.5) (layer "B.Cu") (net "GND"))
 (segment (start 110.731313 73.0208) (end 114.6914 73.0208) (width 1.5) (layer "B.Cu") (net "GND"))
 (segment (start 133.012379 72.939734) (end 133.093445 73.0208) (width 1.5) (layer "B.Cu") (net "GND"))
 (segment (start 114.7044 73.0078) (end 132.944313 73.0078) (width 3) (layer "B.Cu") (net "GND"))
 (segment (start 101.5234 67.8278) (end 106.8304 73.1348) (width 3) (layer "B.Cu") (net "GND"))
 (segment (start 102.5124 61.5778) (end 101.5234 62.5668) (width 3) (layer "B.Cu") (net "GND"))
 (segment (start 101.5234 62.5668) (end 101.5234 67.8278) (width 3) (layer "B.Cu") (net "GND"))
 (segment (start 110.617313 73.1348) (end 110.662379 73.089734) (width 3) (layer "B.Cu") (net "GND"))
 (segment (start 136.7659 73.0208) (end 137.9454 71.8413) (width 1.5) (layer "B.Cu") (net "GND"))
 (segment (start 135.0384 53.2728) (end 134.9204 53.3908) (width 1.5) (layer "F.Cu") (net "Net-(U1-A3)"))
 (segment (start 135.3679 53.2728) (end 135.3524 53.2883) (width 1.5) (layer "F.Cu") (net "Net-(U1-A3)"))
 (segment (start 137.9454 53.2728) (end 135.0384 53.2728) (width 1.5) (layer "F.Cu") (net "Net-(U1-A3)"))
 (segment (start 137.9454 54.8233) (end 137.9454 53.2728) (width 1.5) (layer "F.Cu") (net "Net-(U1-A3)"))
 (segment (start 84.64 74) (end 91.4 74) (width 1.5) (layer "F.Cu") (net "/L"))
 (segment (start 86.614 89.535) (end 91.44 84.709) (width 1.5) (layer "F.Cu") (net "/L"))
 (segment (start 91.44 74.04) (end 91.4 74) (width 1.5) (layer "F.Cu") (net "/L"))
 (segment (start 83.058 89.535) (end 86.614 89.535) (width 1.5) (layer "F.Cu") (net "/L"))
 (segment (start 91.44 84.709) (end 91.44 74.04) (width 1.5) (layer "F.Cu") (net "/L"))
 (segment (start 73.675 70.925) (end 73.675 70.315) (width 1.5) (layer "F.Cu") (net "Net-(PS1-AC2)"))
 (segment (start 81.475 64.825) (end 83.4 66.75) (width 1.5) (layer "F.Cu") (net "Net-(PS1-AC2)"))
 (segment (start 73.675 70.315) (end 73.675 64.825) (width 1.5) (layer "F.Cu") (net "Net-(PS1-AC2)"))
 (segment (start 70.6 74) (end 73.675 70.925) (width 1.5) (layer "F.Cu") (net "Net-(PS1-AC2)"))
 (segment (start 77.36 78.19) (end 76.05 79.5) (width 1.5) (layer "F.Cu") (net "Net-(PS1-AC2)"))
 (segment (start 77.36 74) (end 77.36 78.19) (width 1.5) (layer "F.Cu") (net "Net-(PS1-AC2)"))
 (segment (start 73.675 64.825) (end 81.475 64.825) (width 1.5) (layer "F.Cu") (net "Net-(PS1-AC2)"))
 (segment (start 77.36 74) (end 73.675 70.315) (width 1.5) (layer "F.Cu") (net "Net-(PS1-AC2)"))
 (segment (start 55.65 86.5) (end 53.65 84.5) (width 1.5) (layer "F.Cu") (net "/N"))
 (segment (start 78.058 89.535) (end 78.058 86.487) (width 1.5) (layer "F.Cu") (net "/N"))
 (segment (start 81 80.7825) (end 81 70.5) (width 1.5) (layer "F.Cu") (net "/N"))
 (segment (start 81 70.5) (end 77.25 66.75) (width 1.5) (layer "F.Cu") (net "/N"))
 (segment (start 78.045 86.5) (end 78.058 86.487) (width 1.5) (layer "F.Cu") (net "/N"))
 (segment (start 77.25 66.75) (end 75.6 66.75) (width 1.5) (layer "F.Cu") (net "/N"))
 (segment (start 55.65 86.5) (end 78.045 86.5) (width 1.5) (layer "F.Cu") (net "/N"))
 (segment (start 78.058 86.487) (end 78.058 83.7245) (width 1.5) (layer "F.Cu") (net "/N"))
 (segment (start 78.058 83.7245) (end 81 80.7825) (width 1.5) (layer "F.Cu") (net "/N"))
 (segment (start 69.95 79.5) (end 69.95 80.9) (width 1.5) (layer "F.Cu") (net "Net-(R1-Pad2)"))
 (segment (start 69.95 80.9) (end 66.35 84.5) (width 1.5) (layer "F.Cu") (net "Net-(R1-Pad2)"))
 (segment (start 136.7659 73.0208) (end 137.9454 71.8413) (width 1.5) (layer "F.Cu") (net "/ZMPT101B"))
 (segment (start 107.156481 73.0208) (end 136.7659 73.0208) (width 1.5) (layer "F.Cu") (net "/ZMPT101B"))
 (segment (start 52.47 66.08) (end 49.5 66.08) (width 1) (layer "F.Cu") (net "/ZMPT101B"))
 (segment (start 100.175481 66.0398) (end 98.9734 66.0398) (width 1.5) (layer "F.Cu") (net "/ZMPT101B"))
 (segment (start 100.175481 66.0398) (end 107.156481 73.0208) (width 1.5) (layer "F.Cu") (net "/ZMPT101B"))
 (segment (start 60.65 64) (end 59.6 64) (width 1) (layer "F.Cu") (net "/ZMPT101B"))
 (segment (start 61.1875 64) (end 60.65 64) (width 1) (layer "F.Cu") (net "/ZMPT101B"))
 (segment (start 58.6 66.05) (end 52.5 66.05) (width 1) (layer "F.Cu") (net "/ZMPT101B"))
 (segment (start 52.5 66.05) (end 52.47 66.08) (width 1) (layer "F.Cu") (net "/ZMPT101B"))
 (segment (start 137.9454 56.6483) (end 137.9454 71.8413) (width 1.5) (layer "F.Cu") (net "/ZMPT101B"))
 (segment (start 60.65 64) (end 58.6 66.05) (width 1) (layer "F.Cu") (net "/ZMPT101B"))
 (segment (start 61.2 65.5875) (end 61.2 64.0125) (width 1) (layer "F.Cu") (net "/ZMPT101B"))
 (segment (start 61.2 64.0125) (end 61.1875 64) (width 1) (layer "F.Cu") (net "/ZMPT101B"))
 (segment (start 49.5 63.54) (end 48.44 63.54) (width 1.5) (layer "F.Cu") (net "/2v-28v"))
 (segment (start 48.44 63.54) (end 47.45 62.55) (width 1.5) (layer "F.Cu") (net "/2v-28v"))
 (segment (start 47.45 58.522375) (end 47.45 62.55) (width 1.5) (layer "F.Cu") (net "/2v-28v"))
 (segment (start 51.412375 56.075) (end 49.897375 56.075) (width 1.5) (layer "F.Cu") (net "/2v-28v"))
 (segment (start 49.897375 56.075) (end 47.45 58.522375) (width 1.5) (layer "F.Cu") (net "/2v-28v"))
 (segment (start 63.05 63.9625) (end 63.0125 64) (width 1) (layer "F.Cu") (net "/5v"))
 (segment (start 63.05 62.45) (end 63.05 63.9625) (width 1) (layer "F.Cu") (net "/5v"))
 (segment (start 96.9244 21.9538) (end 118.7234 21.9538) (width 1.5) (layer "F.Cu") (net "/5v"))
 (segment (start 90.8 24.25) (end 86.825 20.275) (width 1.5) (layer "F.Cu") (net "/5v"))
 (segment (start 118.7234 21.9538) (end 134.9204 38.1508) (width 1.5) (layer "F.Cu") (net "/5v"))
 (segment (start 96.9244 66.536385) (end 96.9244 21.9538) (width 1.5) (layer "F.Cu") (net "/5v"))
 (segment (start 55.662375 20.275) (end 51.412375 24.525) (width 1.5) (layer "F.Cu") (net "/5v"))
 (segment (start 98.967815 68.5798) (end 96.9244 66.536385) (width 1.5) (layer "F.Cu") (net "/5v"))
 (segment (start 86.825 20.275) (end 55.662375 20.275) (width 1.5) (layer "F.Cu") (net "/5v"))
 (segment (start 63.05 62.45) (end 58.764178 62.45) (width 1) (layer "F.Cu") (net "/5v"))
 (segment (start 98.9734 68.5798) (end 98.967815 68.5798) (width 1.5) (layer "F.Cu") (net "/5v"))
 (via (at 58.669589 62.544589) (size 0.6) (drill 0.3) (layers "F.Cu" "B.Cu") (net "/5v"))
 (segment (start 90.8 30.414178) (end 58.764178 62.45) (width 1.5) (layer "B.Cu") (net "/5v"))
 (segment (start 90.8 24.25) (end 90.8 30.414178) (width 1.5) (layer "B.Cu") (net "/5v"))
 (segment (start 58.764178 62.45) (end 52.594178 68.62) (width 1.5) (layer "B.Cu") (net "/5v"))
 (segment (start 52.594178 68.62) (end 49.5 68.62) (width 1.5) (layer "B.Cu") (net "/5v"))
 (segment (start 61.25 68.9) (end 61.25 67.3625) (width 1) (layer "F.Cu") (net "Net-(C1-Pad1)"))
 (segment (start 61.25 67.3625) (end 61.2 67.3125) (width 1) (layer "F.Cu") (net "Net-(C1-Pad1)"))
 (segment (start 61.25 69.4) (end 61.25 68.9) (width 1) (layer "F.Cu") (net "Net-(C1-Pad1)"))
 (segment (start 61.25 69.4) (end 66.35 74.5) (width 1) (layer "F.Cu") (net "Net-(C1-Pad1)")))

